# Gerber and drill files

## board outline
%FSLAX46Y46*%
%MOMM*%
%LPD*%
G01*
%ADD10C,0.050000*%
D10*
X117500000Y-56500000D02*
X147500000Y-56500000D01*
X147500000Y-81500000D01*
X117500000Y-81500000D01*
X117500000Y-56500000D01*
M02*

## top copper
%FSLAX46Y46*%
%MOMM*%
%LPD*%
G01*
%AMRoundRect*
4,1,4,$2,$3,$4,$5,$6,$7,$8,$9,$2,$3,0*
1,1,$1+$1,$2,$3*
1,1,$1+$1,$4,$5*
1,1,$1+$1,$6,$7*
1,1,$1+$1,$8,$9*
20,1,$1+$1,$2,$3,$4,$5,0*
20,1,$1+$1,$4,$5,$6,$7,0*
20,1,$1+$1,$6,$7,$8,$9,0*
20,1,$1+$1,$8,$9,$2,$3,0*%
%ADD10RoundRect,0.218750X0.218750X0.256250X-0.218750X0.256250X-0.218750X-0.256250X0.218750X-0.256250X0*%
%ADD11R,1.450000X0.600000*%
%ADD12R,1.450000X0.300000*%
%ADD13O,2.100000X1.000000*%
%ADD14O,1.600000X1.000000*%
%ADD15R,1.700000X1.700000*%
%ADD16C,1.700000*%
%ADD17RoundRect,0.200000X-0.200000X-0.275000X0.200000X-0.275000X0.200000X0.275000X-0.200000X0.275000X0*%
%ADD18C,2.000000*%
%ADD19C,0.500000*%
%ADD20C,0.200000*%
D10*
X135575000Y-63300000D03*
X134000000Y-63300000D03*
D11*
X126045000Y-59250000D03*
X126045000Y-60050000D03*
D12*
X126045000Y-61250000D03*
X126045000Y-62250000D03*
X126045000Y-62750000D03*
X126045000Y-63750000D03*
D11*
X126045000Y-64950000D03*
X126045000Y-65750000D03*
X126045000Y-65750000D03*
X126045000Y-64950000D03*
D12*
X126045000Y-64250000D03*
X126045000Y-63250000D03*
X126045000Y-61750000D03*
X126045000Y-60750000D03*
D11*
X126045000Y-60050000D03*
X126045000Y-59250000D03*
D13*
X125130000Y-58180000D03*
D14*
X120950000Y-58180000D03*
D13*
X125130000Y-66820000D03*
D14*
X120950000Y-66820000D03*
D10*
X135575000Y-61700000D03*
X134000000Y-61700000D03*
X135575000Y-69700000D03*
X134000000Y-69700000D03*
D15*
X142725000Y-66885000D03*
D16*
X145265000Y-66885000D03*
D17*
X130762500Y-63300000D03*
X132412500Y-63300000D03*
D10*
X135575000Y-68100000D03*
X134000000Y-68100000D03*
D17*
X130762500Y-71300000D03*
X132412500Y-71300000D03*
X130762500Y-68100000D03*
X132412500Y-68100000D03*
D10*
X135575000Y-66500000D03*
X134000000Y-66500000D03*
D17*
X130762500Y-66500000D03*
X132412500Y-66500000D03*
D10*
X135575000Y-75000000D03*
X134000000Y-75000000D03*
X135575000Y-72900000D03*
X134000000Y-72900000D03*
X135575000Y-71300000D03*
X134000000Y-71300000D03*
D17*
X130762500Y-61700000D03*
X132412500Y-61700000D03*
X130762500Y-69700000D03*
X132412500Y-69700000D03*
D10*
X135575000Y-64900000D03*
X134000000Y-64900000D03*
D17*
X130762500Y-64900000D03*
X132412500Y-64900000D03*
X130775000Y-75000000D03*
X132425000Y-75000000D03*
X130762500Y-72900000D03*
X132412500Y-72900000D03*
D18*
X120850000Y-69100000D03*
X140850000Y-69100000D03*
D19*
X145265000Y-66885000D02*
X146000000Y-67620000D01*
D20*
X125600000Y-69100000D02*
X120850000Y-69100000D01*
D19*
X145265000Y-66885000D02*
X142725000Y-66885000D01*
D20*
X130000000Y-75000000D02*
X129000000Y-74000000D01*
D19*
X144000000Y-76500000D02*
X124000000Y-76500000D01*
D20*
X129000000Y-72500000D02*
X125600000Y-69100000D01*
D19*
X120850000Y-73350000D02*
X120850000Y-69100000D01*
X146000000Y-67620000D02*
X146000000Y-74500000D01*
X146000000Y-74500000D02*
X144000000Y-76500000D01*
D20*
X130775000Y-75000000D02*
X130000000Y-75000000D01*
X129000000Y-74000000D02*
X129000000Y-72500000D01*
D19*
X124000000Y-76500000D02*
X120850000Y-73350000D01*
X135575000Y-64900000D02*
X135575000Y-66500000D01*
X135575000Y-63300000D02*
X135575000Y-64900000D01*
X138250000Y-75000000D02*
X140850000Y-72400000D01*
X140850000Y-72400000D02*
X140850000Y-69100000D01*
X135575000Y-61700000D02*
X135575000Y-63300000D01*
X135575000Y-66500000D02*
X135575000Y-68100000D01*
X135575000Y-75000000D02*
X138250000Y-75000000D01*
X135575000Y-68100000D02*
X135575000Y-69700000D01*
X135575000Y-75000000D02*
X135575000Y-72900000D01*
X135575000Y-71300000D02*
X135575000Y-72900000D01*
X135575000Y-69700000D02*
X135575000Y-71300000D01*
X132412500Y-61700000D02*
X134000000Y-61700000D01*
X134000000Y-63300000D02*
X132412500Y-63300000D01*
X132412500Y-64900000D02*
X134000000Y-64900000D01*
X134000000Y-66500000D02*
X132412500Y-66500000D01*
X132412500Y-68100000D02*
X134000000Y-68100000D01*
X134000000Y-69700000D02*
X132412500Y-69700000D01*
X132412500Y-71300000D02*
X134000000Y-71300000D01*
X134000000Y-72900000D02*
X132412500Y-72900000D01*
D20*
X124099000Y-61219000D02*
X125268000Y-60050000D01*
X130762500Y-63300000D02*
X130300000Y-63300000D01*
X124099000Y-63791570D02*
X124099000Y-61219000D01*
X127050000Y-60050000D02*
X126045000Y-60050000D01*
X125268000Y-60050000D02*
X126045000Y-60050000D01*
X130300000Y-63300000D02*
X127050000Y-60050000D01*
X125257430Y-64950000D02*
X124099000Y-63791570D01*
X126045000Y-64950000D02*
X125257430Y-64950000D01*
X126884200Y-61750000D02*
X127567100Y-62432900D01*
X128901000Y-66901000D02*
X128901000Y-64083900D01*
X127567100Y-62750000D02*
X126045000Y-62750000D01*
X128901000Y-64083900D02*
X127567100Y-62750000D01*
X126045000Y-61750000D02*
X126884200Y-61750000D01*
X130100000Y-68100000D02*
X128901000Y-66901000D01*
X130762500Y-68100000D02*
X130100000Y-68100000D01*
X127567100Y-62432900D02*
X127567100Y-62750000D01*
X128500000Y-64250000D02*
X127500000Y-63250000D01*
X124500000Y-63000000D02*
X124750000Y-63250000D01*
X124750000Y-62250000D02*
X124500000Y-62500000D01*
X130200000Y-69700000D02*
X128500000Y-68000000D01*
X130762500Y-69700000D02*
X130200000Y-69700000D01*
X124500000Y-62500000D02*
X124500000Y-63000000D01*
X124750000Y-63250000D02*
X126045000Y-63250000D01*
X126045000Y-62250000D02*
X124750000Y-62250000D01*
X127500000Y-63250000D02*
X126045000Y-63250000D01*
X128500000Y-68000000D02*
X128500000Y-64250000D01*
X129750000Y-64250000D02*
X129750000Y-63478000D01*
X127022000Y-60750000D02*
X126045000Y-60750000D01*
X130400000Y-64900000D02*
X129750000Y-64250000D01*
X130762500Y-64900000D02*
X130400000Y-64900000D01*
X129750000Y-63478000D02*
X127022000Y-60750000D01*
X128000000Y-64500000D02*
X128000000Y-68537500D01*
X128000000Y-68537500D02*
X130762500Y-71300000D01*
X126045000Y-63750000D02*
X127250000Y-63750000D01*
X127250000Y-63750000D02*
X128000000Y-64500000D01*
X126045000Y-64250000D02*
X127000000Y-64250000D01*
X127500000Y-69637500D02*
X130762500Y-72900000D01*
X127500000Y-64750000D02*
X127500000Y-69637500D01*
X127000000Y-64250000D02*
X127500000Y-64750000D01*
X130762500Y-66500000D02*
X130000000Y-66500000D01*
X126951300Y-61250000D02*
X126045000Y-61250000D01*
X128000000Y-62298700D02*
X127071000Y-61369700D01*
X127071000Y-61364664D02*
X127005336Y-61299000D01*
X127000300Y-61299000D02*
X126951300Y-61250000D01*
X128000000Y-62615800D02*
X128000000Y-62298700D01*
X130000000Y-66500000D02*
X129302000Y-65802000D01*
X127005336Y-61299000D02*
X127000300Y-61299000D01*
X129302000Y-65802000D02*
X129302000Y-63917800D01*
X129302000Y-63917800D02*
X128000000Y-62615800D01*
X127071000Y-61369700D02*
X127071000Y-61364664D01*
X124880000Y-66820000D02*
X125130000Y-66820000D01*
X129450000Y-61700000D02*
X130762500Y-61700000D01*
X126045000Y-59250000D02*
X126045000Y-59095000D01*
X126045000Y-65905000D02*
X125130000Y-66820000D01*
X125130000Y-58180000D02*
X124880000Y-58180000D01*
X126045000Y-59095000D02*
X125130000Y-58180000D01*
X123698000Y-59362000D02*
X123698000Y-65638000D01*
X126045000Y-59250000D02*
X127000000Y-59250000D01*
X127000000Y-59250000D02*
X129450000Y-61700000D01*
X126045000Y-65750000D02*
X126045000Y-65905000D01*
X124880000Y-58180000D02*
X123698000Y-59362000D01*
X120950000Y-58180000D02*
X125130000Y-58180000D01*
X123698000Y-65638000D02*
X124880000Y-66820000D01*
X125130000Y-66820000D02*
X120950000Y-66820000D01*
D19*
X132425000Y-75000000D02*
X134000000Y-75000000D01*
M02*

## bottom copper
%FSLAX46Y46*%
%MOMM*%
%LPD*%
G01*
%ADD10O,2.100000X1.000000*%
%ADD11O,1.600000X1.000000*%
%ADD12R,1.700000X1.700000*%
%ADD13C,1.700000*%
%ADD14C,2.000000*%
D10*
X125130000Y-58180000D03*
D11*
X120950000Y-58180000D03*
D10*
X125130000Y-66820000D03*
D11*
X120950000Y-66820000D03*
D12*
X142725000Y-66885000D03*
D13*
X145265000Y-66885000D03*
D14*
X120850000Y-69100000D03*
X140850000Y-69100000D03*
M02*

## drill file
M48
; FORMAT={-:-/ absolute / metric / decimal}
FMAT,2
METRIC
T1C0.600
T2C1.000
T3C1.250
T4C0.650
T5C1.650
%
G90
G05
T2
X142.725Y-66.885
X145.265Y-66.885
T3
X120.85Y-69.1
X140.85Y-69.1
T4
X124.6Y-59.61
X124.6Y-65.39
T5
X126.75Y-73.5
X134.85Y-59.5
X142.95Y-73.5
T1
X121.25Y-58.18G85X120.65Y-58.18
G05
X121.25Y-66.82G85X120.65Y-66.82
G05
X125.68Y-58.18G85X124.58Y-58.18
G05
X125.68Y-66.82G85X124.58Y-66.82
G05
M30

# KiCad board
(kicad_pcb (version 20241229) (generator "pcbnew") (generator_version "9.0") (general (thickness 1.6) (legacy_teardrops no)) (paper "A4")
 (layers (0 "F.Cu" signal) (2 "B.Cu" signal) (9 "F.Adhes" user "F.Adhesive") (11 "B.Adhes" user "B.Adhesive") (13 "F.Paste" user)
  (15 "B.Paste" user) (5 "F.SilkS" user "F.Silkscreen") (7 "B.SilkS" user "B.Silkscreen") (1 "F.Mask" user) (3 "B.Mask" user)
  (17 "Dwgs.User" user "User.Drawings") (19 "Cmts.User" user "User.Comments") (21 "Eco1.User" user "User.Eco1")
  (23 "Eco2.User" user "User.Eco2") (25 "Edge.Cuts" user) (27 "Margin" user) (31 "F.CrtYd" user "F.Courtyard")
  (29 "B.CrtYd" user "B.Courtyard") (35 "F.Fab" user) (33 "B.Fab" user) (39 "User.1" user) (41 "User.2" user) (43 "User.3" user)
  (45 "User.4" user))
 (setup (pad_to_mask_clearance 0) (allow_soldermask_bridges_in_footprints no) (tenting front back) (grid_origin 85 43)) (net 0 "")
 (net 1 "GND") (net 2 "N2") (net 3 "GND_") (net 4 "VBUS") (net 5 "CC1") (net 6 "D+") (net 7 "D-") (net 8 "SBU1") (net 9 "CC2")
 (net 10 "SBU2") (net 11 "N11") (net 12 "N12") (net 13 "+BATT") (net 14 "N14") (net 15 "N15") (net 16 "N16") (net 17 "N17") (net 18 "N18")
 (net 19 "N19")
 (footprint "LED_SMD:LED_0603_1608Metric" (layer "F.Cu") (at 134.7875 63.3 180)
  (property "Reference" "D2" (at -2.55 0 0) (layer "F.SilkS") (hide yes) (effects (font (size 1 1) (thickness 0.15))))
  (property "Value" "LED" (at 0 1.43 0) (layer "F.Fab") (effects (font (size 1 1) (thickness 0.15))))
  (pad "1" smd roundrect (at -0.7875 0 180) (size 0.875 0.95) (layers "F.Cu" "F.Mask" "F.Paste") (roundrect_rratio 0.25) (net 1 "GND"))
  (pad "2" smd roundrect (at 0.7875 0 180) (size 0.875 0.95) (layers "F.Cu" "F.Mask" "F.Paste") (roundrect_rratio 0.25) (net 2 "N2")))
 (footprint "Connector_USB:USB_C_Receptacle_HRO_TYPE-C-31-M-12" (layer "F.Cu") (at 122 62.5 -90)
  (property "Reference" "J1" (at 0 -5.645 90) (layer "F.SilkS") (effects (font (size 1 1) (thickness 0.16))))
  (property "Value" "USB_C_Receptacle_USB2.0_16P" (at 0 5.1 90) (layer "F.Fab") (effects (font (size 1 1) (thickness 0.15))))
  (pad "" np_thru_hole circle (at -2.89 -2.6 270) (size 0.65 0.65) (drill 0.65) (layers "*.Cu" "*.Mask"))
  (pad "" np_thru_hole circle (at 2.89 -2.6 270) (size 0.65 0.65) (drill 0.65) (layers "*.Cu" "*.Mask"))
  (pad "A1" smd rect (at -3.25 -4.045 270) (size 0.6 1.45) (layers "F.Cu" "F.Mask" "F.Paste") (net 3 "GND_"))
  (pad "A4" smd rect (at -2.45 -4.045 270) (size 0.6 1.45) (layers "F.Cu" "F.Mask" "F.Paste") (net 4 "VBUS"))
  (pad "A5" smd rect (at -1.25 -4.045 270) (size 0.3 1.45) (layers "F.Cu" "F.Mask" "F.Paste") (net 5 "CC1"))
  (pad "A6" smd rect (at -0.25 -4.045 270) (size 0.3 1.45) (layers "F.Cu" "F.Mask" "F.Paste") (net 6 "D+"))
  (pad "A7" smd rect (at 0.25 -4.045 270) (size 0.3 1.45) (layers "F.Cu" "F.Mask" "F.Paste") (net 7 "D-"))
  (pad "A8" smd rect (at 1.25 -4.045 270) (size 0.3 1.45) (layers "F.Cu" "F.Mask" "F.Paste") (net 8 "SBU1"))
  (pad "A9" smd rect (at 2.45 -4.045 270) (size 0.6 1.45) (layers "F.Cu" "F.Mask" "F.Paste") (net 4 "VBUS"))
  (pad "A12" smd rect (at 3.25 -4.045 270) (size 0.6 1.45) (layers "F.Cu" "F.Mask" "F.Paste") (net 3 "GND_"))
  (pad "B1" smd rect (at 3.25 -4.045 270) (size 0.6 1.45) (layers "F.Cu" "F.Mask" "F.Paste") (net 3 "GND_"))
  (pad "B4" smd rect (at 2.45 -4.045 270) (size 0.6 1.45) (layers "F.Cu" "F.Mask" "F.Paste") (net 4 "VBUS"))
  (pad "B5" smd rect (at 1.75 -4.045 270) (size 0.3 1.45) (layers "F.Cu" "F.Mask" "F.Paste") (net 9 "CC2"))
  (pad "B6" smd rect (at 0.75 -4.045 270) (size 0.3 1.45) (layers "F.Cu" "F.Mask" "F.Paste") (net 6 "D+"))
  (pad "B7" smd rect (at -0.75 -4.045 270) (size 0.3 1.45) (layers "F.Cu" "F.Mask" "F.Paste") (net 7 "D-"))
  (pad "B8" smd rect (at -1.75 -4.045 270) (size 0.3 1.45) (layers "F.Cu" "F.Mask" "F.Paste") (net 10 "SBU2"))
  (pad "B9" smd rect (at -2.45 -4.045 270) (size 0.6 1.45) (layers "F.Cu" "F.Mask" "F.Paste") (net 4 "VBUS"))
  (pad "B12" smd rect (at -3.25 -4.045 270) (size 0.6 1.45) (layers "F.Cu" "F.Mask" "F.Paste") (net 3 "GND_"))
  (pad "S1" thru_hole oval (at -4.32 -3.13 270) (size 1 2.1) (drill oval 0.6 1.7) (layers "*.Cu" "*.Mask") (remove_unused_layers no)
   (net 3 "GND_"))
  (pad "S1" thru_hole oval (at -4.32 1.05 270) (size 1 1.6) (drill oval 0.6 1.2) (layers "*.Cu" "*.Mask") (remove_unused_layers no)
   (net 3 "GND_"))
  (pad "S1" thru_hole oval (at 4.32 -3.13 270) (size 1 2.1) (drill oval 0.6 1.7) (layers "*.Cu" "*.Mask") (remove_unused_layers no)
   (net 3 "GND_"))
  (pad "S1" thru_hole oval (at 4.32 1.05 270) (size 1 1.6) (drill oval 0.6 1.2) (layers "*.Cu" "*.Mask") (remove_unused_layers no)
   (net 3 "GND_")))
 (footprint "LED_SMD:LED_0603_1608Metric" (layer "F.Cu") (at 134.7875 61.7 180)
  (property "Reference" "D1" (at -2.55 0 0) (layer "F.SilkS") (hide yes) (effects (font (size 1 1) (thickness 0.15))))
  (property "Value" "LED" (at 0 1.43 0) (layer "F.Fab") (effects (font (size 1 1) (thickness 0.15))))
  (pad "1" smd roundrect (at -0.7875 0 180) (size 0.875 0.95) (layers "F.Cu" "F.Mask" "F.Paste") (roundrect_rratio 0.25) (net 1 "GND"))
  (pad "2" smd roundrect (at 0.7875 0 180) (size 0.875 0.95) (layers "F.Cu" "F.Mask" "F.Paste") (roundrect_rratio 0.25) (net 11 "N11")))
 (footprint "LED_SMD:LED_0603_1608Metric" (layer "F.Cu") (at 134.7875 69.7 180)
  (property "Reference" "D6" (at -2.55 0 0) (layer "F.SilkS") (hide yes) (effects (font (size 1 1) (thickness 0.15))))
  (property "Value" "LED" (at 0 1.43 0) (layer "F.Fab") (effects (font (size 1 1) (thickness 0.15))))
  (pad "1" smd roundrect (at -0.7875 0 180) (size 0.875 0.95) (layers "F.Cu" "F.Mask" "F.Paste") (roundrect_rratio 0.25) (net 1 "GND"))
  (pad "2" smd roundrect (at 0.7875 0 180) (size 0.875 0.95) (layers "F.Cu" "F.Mask" "F.Paste") (roundrect_rratio 0.25) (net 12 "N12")))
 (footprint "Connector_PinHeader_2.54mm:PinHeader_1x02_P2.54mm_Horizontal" (layer "F.Cu") (at 142.725 66.885 90)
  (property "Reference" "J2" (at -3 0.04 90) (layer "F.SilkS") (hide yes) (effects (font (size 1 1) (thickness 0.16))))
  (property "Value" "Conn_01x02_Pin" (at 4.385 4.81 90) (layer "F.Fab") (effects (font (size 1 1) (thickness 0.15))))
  (pad "1" thru_hole rect (at 0 0 90) (size 1.7 1.7) (drill 1) (layers "*.Cu" "*.Mask") (remove_unused_layers no) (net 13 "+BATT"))
  (pad "2" thru_hole circle (at 0 2.54 90) (size 1.7 1.7) (drill 1) (layers "*.Cu" "*.Mask") (remove_unused_layers no) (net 13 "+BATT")))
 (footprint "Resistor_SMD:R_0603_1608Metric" (layer "F.Cu") (at 131.5875 63.3)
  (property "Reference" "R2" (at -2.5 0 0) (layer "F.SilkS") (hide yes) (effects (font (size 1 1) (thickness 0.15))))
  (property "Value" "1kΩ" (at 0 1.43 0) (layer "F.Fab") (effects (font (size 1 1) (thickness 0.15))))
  (pad "1" smd roundrect (at -0.825 0) (size 0.8 0.95) (layers "F.Cu" "F.Mask" "F.Paste") (roundrect_rratio 0.25) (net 4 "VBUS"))
  (pad "2" smd roundrect (at 0.825 0) (size 0.8 0.95) (layers "F.Cu" "F.Mask" "F.Paste") (roundrect_rratio 0.25) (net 2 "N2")))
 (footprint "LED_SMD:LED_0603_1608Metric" (layer "F.Cu") (at 134.7875 68.1 180)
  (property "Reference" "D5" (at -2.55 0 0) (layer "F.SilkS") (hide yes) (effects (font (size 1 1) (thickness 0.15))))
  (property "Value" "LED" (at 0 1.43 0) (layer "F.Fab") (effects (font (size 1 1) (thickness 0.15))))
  (pad "1" smd roundrect (at -0.7875 0 180) (size 0.875 0.95) (layers "F.Cu" "F.Mask" "F.Paste") (roundrect_rratio 0.25) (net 1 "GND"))
  (pad "2" smd roundrect (at 0.7875 0 180) (size 0.875 0.95) (layers "F.Cu" "F.Mask" "F.Paste") (roundrect_rratio 0.25) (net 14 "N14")))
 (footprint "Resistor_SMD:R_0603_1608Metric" (layer "F.Cu") (at 131.5875 71.3)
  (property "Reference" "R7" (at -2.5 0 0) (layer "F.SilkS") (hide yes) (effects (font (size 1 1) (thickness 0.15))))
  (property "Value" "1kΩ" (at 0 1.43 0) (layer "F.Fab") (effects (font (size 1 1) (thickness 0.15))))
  (pad "1" smd roundrect (at -0.825 0) (size 0.8 0.95) (layers "F.Cu" "F.Mask" "F.Paste") (roundrect_rratio 0.25) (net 8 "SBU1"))
  (pad "2" smd roundrect (at 0.825 0) (size 0.8 0.95) (layers "F.Cu" "F.Mask" "F.Paste") (roundrect_rratio 0.25) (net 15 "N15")))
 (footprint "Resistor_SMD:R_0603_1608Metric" (layer "F.Cu") (at 131.5875 68.1)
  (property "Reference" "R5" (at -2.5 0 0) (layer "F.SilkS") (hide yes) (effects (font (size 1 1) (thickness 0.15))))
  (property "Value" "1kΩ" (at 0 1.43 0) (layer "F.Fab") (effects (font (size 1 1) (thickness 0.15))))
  (pad "1" smd roundrect (at -0.825 0) (size 0.8 0.95) (layers "F.Cu" "F.Mask" "F.Paste") (roundrect_rratio 0.25) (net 7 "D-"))
  (pad "2" smd roundrect (at 0.825 0) (size 0.8 0.95) (layers "F.Cu" "F.Mask" "F.Paste") (roundrect_rratio 0.25) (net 14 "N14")))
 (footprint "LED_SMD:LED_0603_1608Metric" (layer "F.Cu") (at 134.7875 66.5 180)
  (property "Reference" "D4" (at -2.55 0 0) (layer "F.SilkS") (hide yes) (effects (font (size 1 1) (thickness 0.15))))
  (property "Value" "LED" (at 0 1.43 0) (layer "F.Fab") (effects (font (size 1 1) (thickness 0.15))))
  (pad "1" smd roundrect (at -0.7875 0 180) (size 0.875 0.95) (layers "F.Cu" "F.Mask" "F.Paste") (roundrect_rratio 0.25) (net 1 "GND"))
  (pad "2" smd roundrect (at 0.7875 0 180) (size 0.875 0.95) (layers "F.Cu" "F.Mask" "F.Paste") (roundrect_rratio 0.25) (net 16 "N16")))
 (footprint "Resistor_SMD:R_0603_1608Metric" (layer "F.Cu") (at 131.5875 66.5)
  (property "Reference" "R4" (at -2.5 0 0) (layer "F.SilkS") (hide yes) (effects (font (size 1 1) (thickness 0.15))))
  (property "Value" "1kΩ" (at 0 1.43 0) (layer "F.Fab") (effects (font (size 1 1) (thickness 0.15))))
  (pad "1" smd roundrect (at -0.825 0) (size 0.8 0.95) (layers "F.Cu" "F.Mask" "F.Paste") (roundrect_rratio 0.25) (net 5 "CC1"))
  (pad "2" smd roundrect (at 0.825 0) (size 0.8 0.95) (layers "F.Cu" "F.Mask" "F.Paste") (roundrect_rratio 0.25) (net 16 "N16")))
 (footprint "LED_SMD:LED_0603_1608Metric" (layer "F.Cu") (at 134.7875 75 180)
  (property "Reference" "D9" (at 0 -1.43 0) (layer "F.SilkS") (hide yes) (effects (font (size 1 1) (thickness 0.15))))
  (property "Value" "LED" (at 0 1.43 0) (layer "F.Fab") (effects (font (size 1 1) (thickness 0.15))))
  (pad "1" smd roundrect (at -0.7875 0 180) (size 0.875 0.95) (layers "F.Cu" "F.Mask" "F.Paste") (roundrect_rratio 0.25) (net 1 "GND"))
  (pad "2" smd roundrect (at 0.7875 0 180) (size 0.875 0.95) (layers "F.Cu" "F.Mask" "F.Paste") (roundrect_rratio 0.25) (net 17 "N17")))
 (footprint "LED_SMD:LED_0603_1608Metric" (layer "F.Cu") (at 134.7875 72.9 180)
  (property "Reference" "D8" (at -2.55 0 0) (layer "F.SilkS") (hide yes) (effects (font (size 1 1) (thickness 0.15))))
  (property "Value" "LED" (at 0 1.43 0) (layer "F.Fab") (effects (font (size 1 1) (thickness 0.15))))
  (pad "1" smd roundrect (at -0.7875 0 180) (size 0.875 0.95) (layers "F.Cu" "F.Mask" "F.Paste") (roundrect_rratio 0.25) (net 1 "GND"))
  (pad "2" smd roundrect (at 0.7875 0 180) (size 0.875 0.95) (layers "F.Cu" "F.Mask" "F.Paste") (roundrect_rratio 0.25) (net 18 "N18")))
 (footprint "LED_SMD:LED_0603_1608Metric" (layer "F.Cu") (at 134.7875 71.3 180)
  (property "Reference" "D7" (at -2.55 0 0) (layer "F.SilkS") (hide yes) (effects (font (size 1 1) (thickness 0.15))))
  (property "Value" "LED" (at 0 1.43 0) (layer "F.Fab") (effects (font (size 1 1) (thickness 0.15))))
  (pad "1" smd roundrect (at -0.7875 0 180) (size 0.875 0.95) (layers "F.Cu" "F.Mask" "F.Paste") (roundrect_rratio 0.25) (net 1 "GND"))
  (pad "2" smd roundrect (at 0.7875 0 180) (size 0.875 0.95) (layers "F.Cu" "F.Mask" "F.Paste") (roundrect_rratio 0.25) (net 15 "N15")))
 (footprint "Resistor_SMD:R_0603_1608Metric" (layer "F.Cu") (at 131.5875 61.7)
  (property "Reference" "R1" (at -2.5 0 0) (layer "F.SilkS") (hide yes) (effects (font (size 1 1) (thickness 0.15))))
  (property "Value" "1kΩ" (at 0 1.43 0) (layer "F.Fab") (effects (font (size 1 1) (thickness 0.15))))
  (pad "1" smd roundrect (at -0.825 0) (size 0.8 0.95) (layers "F.Cu" "F.Mask" "F.Paste") (roundrect_rratio 0.25) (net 3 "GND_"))
  (pad "2" smd roundrect (at 0.825 0) (size 0.8 0.95) (layers "F.Cu" "F.Mask" "F.Paste") (roundrect_rratio 0.25) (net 11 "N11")))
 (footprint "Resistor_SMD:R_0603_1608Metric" (layer "F.Cu") (at 131.5875 69.7)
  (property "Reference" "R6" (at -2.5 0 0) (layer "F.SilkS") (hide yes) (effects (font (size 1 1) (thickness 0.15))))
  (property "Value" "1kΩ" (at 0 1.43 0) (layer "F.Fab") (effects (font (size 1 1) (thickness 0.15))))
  (pad "1" smd roundrect (at -0.825 0) (size 0.8 0.95) (layers "F.Cu" "F.Mask" "F.Paste") (roundrect_rratio 0.25) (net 6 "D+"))
  (pad "2" smd roundrect (at 0.825 0) (size 0.8 0.95) (layers "F.Cu" "F.Mask" "F.Paste") (roundrect_rratio 0.25) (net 12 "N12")))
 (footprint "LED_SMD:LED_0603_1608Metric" (layer "F.Cu") (at 134.7875 64.9 180)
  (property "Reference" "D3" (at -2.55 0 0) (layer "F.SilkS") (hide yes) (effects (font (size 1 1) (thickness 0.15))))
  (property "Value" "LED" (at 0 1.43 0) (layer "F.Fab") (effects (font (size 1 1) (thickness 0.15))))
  (pad "1" smd roundrect (at -0.7875 0 180) (size 0.875 0.95) (layers "F.Cu" "F.Mask" "F.Paste") (roundrect_rratio 0.25) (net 1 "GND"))
  (pad "2" smd roundrect (at 0.7875 0 180) (size 0.875 0.95) (layers "F.Cu" "F.Mask" "F.Paste") (roundrect_rratio 0.25) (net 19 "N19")))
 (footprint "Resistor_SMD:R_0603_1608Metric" (layer "F.Cu") (at 131.5875 64.9)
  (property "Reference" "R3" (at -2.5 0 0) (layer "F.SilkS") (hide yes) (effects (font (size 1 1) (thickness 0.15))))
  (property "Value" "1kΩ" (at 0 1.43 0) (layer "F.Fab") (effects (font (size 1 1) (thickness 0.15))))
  (pad "1" smd roundrect (at -0.825 0) (size 0.8 0.95) (layers "F.Cu" "F.Mask" "F.Paste") (roundrect_rratio 0.25) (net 10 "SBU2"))
  (pad "2" smd roundrect (at 0.825 0) (size 0.8 0.95) (layers "F.Cu" "F.Mask" "F.Paste") (roundrect_rratio 0.25) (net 19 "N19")))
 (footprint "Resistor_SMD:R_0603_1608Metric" (layer "F.Cu") (at 131.6 75)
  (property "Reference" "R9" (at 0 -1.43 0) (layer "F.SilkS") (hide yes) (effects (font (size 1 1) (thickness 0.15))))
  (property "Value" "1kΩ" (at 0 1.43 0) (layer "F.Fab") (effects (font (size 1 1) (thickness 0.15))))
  (pad "1" smd roundrect (at -0.825 0) (size 0.8 0.95) (layers "F.Cu" "F.Mask" "F.Paste") (roundrect_rratio 0.25) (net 13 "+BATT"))
  (pad "2" smd roundrect (at 0.825 0) (size 0.8 0.95) (layers "F.Cu" "F.Mask" "F.Paste") (roundrect_rratio 0.25) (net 17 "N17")))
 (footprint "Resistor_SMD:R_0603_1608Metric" (layer "F.Cu") (at 131.5875 72.9)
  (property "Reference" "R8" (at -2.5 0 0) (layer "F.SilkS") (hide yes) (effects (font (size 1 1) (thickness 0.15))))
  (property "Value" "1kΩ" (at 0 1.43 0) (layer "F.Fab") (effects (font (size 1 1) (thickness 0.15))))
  (pad "1" smd roundrect (at -0.825 0) (size 0.8 0.95) (layers "F.Cu" "F.Mask" "F.Paste") (roundrect_rratio 0.25) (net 9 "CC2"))
  (pad "2" smd roundrect (at 0.825 0) (size 0.8 0.95) (layers "F.Cu" "F.Mask" "F.Paste") (roundrect_rratio 0.25) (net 18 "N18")))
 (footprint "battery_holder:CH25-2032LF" (layer "B.Cu") (at 129.85 69.1 90)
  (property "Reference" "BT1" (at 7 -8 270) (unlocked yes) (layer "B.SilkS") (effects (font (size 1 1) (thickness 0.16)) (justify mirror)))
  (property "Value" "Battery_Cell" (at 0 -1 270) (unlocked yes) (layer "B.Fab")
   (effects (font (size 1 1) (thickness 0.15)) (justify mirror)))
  (pad "" np_thru_hole circle (at -4.4 -3.1 90) (size 1.65 1.65) (drill 1.65) (layers "*.Cu" "*.Mask"))
  (pad "" np_thru_hole circle (at -4.4 13.1 90) (size 1.65 1.65) (drill 1.65) (layers "*.Cu" "*.Mask"))
  (pad "" np_thru_hole circle (at 9.6 5 90) (size 1.65 1.65) (drill 1.65) (layers "*.Cu" "*.Mask"))
  (pad "1" thru_hole circle (at 0 -9 90) (size 2 2) (drill 1.25) (layers "*.Cu" "*.Mask") (remove_unused_layers no) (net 13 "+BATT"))
  (pad "2" thru_hole circle (at 0 11 90) (size 2 2) (drill 1.25) (layers "*.Cu" "*.Mask") (remove_unused_layers no) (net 1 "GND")))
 (gr_rect (start 117.5 56.5) (end 147.5 81.5) (stroke (width 0.05) (type default)) (fill no) (layer "Edge.Cuts"))
 (segment (start 145.265 66.885) (end 146 67.62) (width 0.5) (layer "F.Cu") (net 13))
 (segment (start 125.6 69.1) (end 120.85 69.1) (width 0.2) (layer "F.Cu") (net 13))
 (segment (start 145.265 66.885) (end 142.725 66.885) (width 0.5) (layer "F.Cu") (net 13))
 (segment (start 130 75) (end 129 74) (width 0.2) (layer "F.Cu") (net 13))
 (segment (start 144 76.5) (end 124 76.5) (width 0.5) (layer "F.Cu") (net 13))
 (segment (start 129 72.5) (end 125.6 69.1) (width 0.2) (layer "F.Cu") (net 13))
 (segment (start 120.85 73.35) (end 120.85 69.1) (width 0.5) (layer "F.Cu") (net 13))
 (segment (start 146 67.62) (end 146 74.5) (width 0.5) (layer "F.Cu") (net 13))
 (segment (start 146 74.5) (end 144 76.5) (width 0.5) (layer "F.Cu") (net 13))
 (segment (start 130.775 75) (end 130 75) (width 0.2) (layer "F.Cu") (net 13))
 (segment (start 129 74) (end 129 72.5) (width 0.2) (layer "F.Cu") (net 13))
 (segment (start 124 76.5) (end 120.85 73.35) (width 0.5) (layer "F.Cu") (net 13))
 (segment (start 135.575 64.9) (end 135.575 66.5) (width 0.5) (layer "F.Cu") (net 1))
 (segment (start 135.575 63.3) (end 135.575 64.9) (width 0.5) (layer "F.Cu") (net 1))
 (segment (start 138.25 75) (end 140.85 72.4) (width 0.5) (layer "F.Cu") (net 1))
 (segment (start 140.85 72.4) (end 140.85 69.1) (width 0.5) (layer "F.Cu") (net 1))
 (segment (start 135.575 61.7) (end 135.575 63.3) (width 0.5) (layer "F.Cu") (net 1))
 (segment (start 135.575 66.5) (end 135.575 68.1) (width 0.5) (layer "F.Cu") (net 1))
 (segment (start 135.575 75) (end 138.25 75) (width 0.5) (layer "F.Cu") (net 1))
 (segment (start 135.575 68.1) (end 135.575 69.7) (width 0.5) (layer "F.Cu") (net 1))
 (segment (start 135.575 75) (end 135.575 72.9) (width 0.5) (layer "F.Cu") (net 1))
 (segment (start 135.575 71.3) (end 135.575 72.9) (width 0.5) (layer "F.Cu") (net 1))
 (segment (start 135.575 69.7) (end 135.575 71.3) (width 0.5) (layer "F.Cu") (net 1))
 (segment (start 132.4125 61.7) (end 134 61.7) (width 0.5) (layer "F.Cu") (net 11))
 (segment (start 134 63.3) (end 132.4125 63.3) (width 0.5) (layer "F.Cu") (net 2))
 (segment (start 132.4125 64.9) (end 134 64.9) (width 0.5) (layer "F.Cu") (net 19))
 (segment (start 134 66.5) (end 132.4125 66.5) (width 0.5) (layer "F.Cu") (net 16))
 (segment (start 132.4125 68.1) (end 134 68.1) (width 0.5) (layer "F.Cu") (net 14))
 (segment (start 134 69.7) (end 132.4125 69.7) (width 0.5) (layer "F.Cu") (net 12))
 (segment (start 132.4125 71.3) (end 134 71.3) (width 0.5) (layer "F.Cu") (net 15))
 (segment (start 134 72.9) (end 132.4125 72.9) (width 0.5) (layer "F.Cu") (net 18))
 (segment (start 124.099 61.219) (end 125.268 60.05) (width 0.2) (layer "F.Cu") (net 4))
 (segment (start 130.7625 63.3) (end 130.3 63.3) (width 0.2) (layer "F.Cu") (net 4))
 (segment (start 124.099 63.79157) (end 124.099 61.219) (width 0.2) (layer "F.Cu") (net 4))
 (segment (start 127.05 60.05) (end 126.045 60.05) (width 0.2) (layer "F.Cu") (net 4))
 (segment (start 125.268 60.05) (end 126.045 60.05) (width 0.2) (layer "F.Cu") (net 4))
 (segment (start 130.3 63.3) (end 127.05 60.05) (width 0.2) (layer "F.Cu") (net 4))
 (segment (start 125.25743 64.95) (end 124.099 63.79157) (width 0.2) (layer "F.Cu") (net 4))
 (segment (start 126.045 64.95) (end 125.25743 64.95) (width 0.2) (layer "F.Cu") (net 4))
 (segment (start 126.8842 61.75) (end 127.5671 62.4329) (width 0.2) (layer "F.Cu") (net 7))
 (segment (start 128.901 66.901) (end 128.901 64.0839) (width 0.2) (layer "F.Cu") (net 7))
 (segment (start 127.5671 62.75) (end 126.045 62.75) (width 0.2) (layer "F.Cu") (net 7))
 (segment (start 128.901 64.0839) (end 127.5671 62.75) (width 0.2) (layer "F.Cu") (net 7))
 (segment (start 126.045 61.75) (end 126.8842 61.75) (width 0.2) (layer "F.Cu") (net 7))
 (segment (start 130.1 68.1) (end 128.901 66.901) (width 0.2) (layer "F.Cu") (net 7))
 (segment (start 130.7625 68.1) (end 130.1 68.1) (width 0.2) (layer "F.Cu") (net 7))
 (segment (start 127.5671 62.4329) (end 127.5671 62.75) (width 0.2) (layer "F.Cu") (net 7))
 (segment (start 128.5 64.25) (end 127.5 63.25) (width 0.2) (layer "F.Cu") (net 6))
 (segment (start 124.5 63) (end 124.75 63.25) (width 0.2) (layer "F.Cu") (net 6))
 (segment (start 124.75 62.25) (end 124.5 62.5) (width 0.2) (layer "F.Cu") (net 6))
 (segment (start 130.2 69.7) (end 128.5 68) (width 0.2) (layer "F.Cu") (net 6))
 (segment (start 130.7625 69.7) (end 130.2 69.7) (width 0.2) (layer "F.Cu") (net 6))
 (segment (start 124.5 62.5) (end 124.5 63) (width 0.2) (layer "F.Cu") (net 6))
 (segment (start 124.75 63.25) (end 126.045 63.25) (width 0.2) (layer "F.Cu") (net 6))
 (segment (start 126.045 62.25) (end 124.75 62.25) (width 0.2) (layer "F.Cu") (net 6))
 (segment (start 127.5 63.25) (end 126.045 63.25) (width 0.2) (layer "F.Cu") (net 6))
 (segment (start 128.5 68) (end 128.5 64.25) (width 0.2) (layer "F.Cu") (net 6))
 (segment (start 129.75 64.25) (end 129.75 63.478) (width 0.2) (layer "F.Cu") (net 10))
 (segment (start 127.022 60.75) (end 126.045 60.75) (width 0.2) (layer "F.Cu") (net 10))
 (segment (start 130.4 64.9) (end 129.75 64.25) (width 0.2) (layer "F.Cu") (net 10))
 (segment (start 130.7625 64.9) (end 130.4 64.9) (width 0.2) (layer "F.Cu") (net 10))
 (segment (start 129.75 63.478) (end 127.022 60.75) (width 0.2) (layer "F.Cu") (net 10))
 (segment (start 128 64.5) (end 128 68.5375) (width 0.2) (layer "F.Cu") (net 8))
 (segment (start 128 68.5375) (end 130.7625 71.3) (width 0.2) (layer "F.Cu") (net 8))
 (segment (start 126.045 63.75) (end 127.25 63.75) (width 0.2) (layer "F.Cu") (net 8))
 (segment (start 127.25 63.75) (end 128 64.5) (width 0.2) (layer "F.Cu") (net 8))
 (segment (start 126.045 64.25) (end 127 64.25) (width 0.2) (layer "F.Cu") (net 9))
 (segment (start 127.5 69.6375) (end 130.7625 72.9) (width 0.2) (layer "F.Cu") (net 9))
 (segment (start 127.5 64.75) (end 127.5 69.6375) (width 0.2) (layer "F.Cu") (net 9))
 (segment (start 127 64.25) (end 127.5 64.75) (width 0.2) (layer "F.Cu") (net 9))
 (segment (start 130.7625 66.5) (end 130 66.5) (width 0.2) (layer "F.Cu") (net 5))
 (segment (start 126.9513 61.25) (end 126.045 61.25) (width 0.2) (layer "F.Cu") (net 5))
 (segment (start 128 62.2987) (end 127.071 61.3697) (width 0.2) (layer "F.Cu") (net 5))
 (segment (start 127.071 61.364664) (end 127.005336 61.299) (width 0.2) (layer "F.Cu") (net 5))
 (segment (start 127.0003 61.299) (end 126.9513 61.25) (width 0.2) (layer "F.Cu") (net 5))
 (segment (start 128 62.6158) (end 128 62.2987) (width 0.2) (layer "F.Cu") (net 5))
 (segment (start 130 66.5) (end 129.302 65.802) (width 0.2) (layer "F.Cu") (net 5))
 (segment (start 127.005336 61.299) (end 127.0003 61.299) (width 0.2) (layer "F.Cu") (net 5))
 (segment (start 129.302 65.802) (end 129.302 63.9178) (width 0.2) (layer "F.Cu") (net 5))
 (segment (start 129.302 63.9178) (end 128 62.6158) (width 0.2) (layer "F.Cu") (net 5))
 (segment (start 127.071 61.3697) (end 127.071 61.364664) (width 0.2) (layer "F.Cu") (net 5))
 (segment (start 124.88 66.82) (end 125.13 66.82) (width 0.2) (layer "F.Cu") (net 3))
 (segment (start 129.45 61.7) (end 130.7625 61.7) (width 0.2) (layer "F.Cu") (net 3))
 (segment (start 126.045 59.25) (end 126.045 59.095) (width 0.2) (layer "F.Cu") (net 3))
 (segment (start 126.045 65.905) (end 125.13 66.82) (width 0.2) (layer "F.Cu") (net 3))
 (segment (start 125.13 58.18) (end 124.88 58.18) (width 0.2) (layer "F.Cu") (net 3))
 (segment (start 126.045 59.095) (end 125.13 58.18) (width 0.2) (layer "F.Cu") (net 3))
 (segment (start 123.698 59.362) (end 123.698 65.638) (width 0.2) (layer "F.Cu") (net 3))
 (segment (start 126.045 59.25) (end 127 59.25) (width 0.2) (layer "F.Cu") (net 3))
 (segment (start 127 59.25) (end 129.45 61.7) (width 0.2) (layer "F.Cu") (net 3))
 (segment (start 126.045 65.75) (end 126.045 65.905) (width 0.2) (layer "F.Cu") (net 3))
 (segment (start 124.88 58.18) (end 123.698 59.362) (width 0.2) (layer "F.Cu") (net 3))
 (segment (start 120.95 58.18) (end 125.13 58.18) (width 0.2) (layer "F.Cu") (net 3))
 (segment (start 123.698 65.638) (end 124.88 66.82) (width 0.2) (layer "F.Cu") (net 3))
 (segment (start 125.13 66.82) (end 120.95 66.82) (width 0.2) (layer "F.Cu") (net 3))
 (segment (start 132.425 75) (end 134 75) (width 0.5) (layer "F.Cu") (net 17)))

